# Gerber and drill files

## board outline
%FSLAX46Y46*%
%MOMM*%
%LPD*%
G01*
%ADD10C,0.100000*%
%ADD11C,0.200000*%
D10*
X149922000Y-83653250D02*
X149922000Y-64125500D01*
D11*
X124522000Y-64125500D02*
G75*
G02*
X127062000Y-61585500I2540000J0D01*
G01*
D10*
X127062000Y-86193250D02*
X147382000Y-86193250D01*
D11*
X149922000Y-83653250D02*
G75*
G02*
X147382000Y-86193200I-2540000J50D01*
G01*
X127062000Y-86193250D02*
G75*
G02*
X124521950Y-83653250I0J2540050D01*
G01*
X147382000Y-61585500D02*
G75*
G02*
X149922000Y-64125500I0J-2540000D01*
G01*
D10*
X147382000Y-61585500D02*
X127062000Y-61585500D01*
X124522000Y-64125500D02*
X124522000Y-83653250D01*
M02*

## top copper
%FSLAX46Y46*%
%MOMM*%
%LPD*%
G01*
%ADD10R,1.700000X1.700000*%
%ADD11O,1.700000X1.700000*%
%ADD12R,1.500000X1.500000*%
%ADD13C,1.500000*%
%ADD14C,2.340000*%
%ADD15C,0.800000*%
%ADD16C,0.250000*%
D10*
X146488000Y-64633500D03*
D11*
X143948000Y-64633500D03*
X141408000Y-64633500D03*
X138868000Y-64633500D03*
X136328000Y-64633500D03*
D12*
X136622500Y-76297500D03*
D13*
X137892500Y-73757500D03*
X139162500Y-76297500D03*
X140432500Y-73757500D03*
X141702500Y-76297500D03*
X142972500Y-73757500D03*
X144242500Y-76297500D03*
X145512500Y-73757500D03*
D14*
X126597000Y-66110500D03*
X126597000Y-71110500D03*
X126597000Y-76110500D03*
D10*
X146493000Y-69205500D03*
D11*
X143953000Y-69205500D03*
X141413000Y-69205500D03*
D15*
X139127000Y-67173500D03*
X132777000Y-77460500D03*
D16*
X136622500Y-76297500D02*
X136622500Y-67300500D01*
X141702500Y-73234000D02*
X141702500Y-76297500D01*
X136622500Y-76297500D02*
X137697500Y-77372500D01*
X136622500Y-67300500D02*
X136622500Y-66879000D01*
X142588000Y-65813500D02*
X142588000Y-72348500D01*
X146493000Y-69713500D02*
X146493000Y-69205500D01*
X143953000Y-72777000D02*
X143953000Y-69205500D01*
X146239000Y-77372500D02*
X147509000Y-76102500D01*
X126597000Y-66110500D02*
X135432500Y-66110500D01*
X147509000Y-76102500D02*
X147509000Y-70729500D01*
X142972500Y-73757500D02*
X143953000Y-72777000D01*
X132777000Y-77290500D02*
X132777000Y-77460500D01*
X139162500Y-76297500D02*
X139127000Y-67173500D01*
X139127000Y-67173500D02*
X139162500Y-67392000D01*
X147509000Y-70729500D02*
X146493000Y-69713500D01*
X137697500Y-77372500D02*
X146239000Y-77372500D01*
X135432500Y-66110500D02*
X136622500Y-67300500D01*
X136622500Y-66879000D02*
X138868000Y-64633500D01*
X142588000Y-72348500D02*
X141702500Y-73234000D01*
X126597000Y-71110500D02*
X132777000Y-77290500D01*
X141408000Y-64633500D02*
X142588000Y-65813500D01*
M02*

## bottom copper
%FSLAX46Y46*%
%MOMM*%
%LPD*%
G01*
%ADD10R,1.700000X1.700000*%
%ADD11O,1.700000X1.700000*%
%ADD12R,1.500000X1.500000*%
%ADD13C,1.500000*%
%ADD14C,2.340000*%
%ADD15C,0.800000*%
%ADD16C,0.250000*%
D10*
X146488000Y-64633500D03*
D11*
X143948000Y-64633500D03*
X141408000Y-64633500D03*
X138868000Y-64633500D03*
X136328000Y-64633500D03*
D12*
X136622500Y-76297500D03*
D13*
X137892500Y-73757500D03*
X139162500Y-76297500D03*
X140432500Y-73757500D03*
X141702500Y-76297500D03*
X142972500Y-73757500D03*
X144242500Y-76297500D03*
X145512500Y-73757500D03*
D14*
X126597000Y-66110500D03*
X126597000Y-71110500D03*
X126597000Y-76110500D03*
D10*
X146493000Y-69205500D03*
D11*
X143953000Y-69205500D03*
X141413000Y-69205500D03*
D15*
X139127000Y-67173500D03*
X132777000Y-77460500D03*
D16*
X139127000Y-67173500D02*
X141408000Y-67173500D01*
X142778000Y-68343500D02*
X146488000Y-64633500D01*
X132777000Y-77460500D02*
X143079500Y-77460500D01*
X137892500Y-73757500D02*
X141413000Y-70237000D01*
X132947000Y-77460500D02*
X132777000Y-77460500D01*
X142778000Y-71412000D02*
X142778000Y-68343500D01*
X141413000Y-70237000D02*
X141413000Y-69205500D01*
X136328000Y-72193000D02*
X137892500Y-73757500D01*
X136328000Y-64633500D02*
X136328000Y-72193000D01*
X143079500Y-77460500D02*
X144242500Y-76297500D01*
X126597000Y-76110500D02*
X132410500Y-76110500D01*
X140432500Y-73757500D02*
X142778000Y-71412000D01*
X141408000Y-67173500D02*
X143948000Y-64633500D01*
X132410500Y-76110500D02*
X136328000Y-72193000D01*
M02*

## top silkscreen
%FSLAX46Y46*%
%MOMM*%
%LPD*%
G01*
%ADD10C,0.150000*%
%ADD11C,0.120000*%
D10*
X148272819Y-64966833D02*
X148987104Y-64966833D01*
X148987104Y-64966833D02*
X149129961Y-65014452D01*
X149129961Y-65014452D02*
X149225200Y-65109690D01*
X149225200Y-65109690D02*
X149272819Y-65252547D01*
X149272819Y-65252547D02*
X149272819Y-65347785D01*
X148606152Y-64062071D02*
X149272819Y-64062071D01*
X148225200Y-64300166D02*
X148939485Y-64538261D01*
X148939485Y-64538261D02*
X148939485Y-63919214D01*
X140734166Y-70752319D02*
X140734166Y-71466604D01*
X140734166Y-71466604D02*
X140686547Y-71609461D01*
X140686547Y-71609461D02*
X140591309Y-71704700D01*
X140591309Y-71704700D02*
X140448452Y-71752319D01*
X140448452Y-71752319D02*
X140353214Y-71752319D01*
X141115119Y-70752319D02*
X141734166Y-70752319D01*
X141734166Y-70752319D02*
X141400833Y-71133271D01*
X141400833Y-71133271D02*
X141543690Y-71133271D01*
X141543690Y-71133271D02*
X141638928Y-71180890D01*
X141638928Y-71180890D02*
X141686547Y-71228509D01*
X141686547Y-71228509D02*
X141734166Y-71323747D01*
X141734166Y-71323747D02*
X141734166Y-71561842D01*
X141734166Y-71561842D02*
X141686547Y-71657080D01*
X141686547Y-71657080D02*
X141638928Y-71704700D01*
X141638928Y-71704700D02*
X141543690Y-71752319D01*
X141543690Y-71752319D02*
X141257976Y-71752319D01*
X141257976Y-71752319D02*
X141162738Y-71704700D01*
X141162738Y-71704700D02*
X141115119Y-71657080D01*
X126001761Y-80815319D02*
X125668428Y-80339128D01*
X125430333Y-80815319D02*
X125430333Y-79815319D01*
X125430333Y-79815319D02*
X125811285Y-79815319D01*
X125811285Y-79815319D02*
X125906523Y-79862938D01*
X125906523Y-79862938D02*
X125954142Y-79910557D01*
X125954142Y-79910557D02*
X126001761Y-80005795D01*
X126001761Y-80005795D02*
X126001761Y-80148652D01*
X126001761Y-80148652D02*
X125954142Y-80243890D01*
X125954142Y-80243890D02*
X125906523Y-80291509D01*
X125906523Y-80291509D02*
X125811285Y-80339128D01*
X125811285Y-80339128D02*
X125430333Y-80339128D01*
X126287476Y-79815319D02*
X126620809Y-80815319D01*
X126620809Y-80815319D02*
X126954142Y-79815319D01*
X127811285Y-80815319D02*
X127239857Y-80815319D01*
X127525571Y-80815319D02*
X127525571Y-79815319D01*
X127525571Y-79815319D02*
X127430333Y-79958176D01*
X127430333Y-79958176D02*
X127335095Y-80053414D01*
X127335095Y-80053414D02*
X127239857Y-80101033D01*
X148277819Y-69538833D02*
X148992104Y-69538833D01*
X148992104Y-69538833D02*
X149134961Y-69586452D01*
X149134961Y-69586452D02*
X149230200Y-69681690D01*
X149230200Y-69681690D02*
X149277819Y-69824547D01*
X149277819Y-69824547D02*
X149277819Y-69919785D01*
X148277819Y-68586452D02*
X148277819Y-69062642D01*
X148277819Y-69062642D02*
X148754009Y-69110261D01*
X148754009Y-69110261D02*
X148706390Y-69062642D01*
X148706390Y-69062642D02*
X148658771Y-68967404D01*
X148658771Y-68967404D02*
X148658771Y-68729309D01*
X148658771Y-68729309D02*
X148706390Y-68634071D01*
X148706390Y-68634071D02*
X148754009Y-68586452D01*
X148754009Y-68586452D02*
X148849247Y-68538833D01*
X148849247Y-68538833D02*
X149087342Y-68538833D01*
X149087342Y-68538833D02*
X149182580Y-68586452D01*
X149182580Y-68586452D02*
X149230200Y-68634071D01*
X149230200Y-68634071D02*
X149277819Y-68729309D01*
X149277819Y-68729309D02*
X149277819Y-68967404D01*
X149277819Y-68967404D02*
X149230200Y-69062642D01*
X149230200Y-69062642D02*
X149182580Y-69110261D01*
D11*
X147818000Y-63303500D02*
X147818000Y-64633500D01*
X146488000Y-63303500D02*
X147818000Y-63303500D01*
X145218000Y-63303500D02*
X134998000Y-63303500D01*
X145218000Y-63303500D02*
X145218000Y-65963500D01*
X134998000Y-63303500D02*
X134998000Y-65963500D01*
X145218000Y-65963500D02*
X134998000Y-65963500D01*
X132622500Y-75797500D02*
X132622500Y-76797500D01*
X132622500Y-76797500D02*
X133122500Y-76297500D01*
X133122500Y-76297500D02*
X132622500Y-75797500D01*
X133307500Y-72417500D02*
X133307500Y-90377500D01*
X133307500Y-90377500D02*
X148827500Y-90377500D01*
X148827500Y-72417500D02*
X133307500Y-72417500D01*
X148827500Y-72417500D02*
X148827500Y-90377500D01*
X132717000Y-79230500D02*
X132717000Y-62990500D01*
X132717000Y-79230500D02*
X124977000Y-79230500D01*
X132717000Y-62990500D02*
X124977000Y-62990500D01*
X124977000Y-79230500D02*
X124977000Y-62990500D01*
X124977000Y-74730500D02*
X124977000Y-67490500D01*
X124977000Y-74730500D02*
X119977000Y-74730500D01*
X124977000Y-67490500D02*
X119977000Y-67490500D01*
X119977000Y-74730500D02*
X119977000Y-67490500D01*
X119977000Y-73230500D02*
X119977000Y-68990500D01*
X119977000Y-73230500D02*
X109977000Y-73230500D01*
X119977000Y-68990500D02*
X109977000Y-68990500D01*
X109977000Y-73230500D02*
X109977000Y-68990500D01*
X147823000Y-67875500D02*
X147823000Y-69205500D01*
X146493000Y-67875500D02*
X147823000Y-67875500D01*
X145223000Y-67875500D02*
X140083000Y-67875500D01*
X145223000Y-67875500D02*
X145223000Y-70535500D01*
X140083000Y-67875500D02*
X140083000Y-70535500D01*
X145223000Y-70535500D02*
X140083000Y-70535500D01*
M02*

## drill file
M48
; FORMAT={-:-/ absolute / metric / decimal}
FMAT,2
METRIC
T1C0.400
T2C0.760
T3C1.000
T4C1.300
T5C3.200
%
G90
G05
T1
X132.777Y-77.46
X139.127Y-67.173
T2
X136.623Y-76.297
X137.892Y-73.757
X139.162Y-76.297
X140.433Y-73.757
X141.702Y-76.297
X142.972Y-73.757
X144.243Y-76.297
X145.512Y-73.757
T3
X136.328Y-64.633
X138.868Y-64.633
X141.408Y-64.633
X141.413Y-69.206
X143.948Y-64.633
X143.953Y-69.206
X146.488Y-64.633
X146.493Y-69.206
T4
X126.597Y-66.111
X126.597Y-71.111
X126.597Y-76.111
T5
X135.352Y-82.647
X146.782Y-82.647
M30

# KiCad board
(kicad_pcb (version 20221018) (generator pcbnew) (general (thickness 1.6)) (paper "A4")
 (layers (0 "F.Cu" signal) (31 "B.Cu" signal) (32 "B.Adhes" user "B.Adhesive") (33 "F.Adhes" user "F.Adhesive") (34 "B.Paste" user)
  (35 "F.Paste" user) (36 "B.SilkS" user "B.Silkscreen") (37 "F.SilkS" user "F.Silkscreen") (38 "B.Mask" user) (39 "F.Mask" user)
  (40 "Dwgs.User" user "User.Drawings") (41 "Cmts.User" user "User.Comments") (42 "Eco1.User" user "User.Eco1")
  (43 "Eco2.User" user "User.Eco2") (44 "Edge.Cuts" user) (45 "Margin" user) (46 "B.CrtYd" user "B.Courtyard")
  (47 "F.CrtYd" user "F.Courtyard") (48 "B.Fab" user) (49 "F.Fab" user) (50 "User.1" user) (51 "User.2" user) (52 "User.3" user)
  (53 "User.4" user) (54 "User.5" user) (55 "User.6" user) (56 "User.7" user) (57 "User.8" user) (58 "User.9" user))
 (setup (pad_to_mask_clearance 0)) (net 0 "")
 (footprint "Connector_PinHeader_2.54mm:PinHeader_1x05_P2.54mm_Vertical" (layer "F.Cu") (at 146.488 64.6335 -90)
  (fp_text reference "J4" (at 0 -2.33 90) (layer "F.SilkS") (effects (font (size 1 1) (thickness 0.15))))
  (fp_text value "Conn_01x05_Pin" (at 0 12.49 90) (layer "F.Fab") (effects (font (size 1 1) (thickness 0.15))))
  (fp_line (start -1.33 -1.33) (end 0 -1.33) (stroke (width 0.12) (type solid)) (layer "F.SilkS"))
  (fp_line (start -1.33 0) (end -1.33 -1.33) (stroke (width 0.12) (type solid)) (layer "F.SilkS"))
  (fp_line (start -1.33 1.27) (end -1.33 11.49) (stroke (width 0.12) (type solid)) (layer "F.SilkS"))
  (fp_line (start -1.33 1.27) (end 1.33 1.27) (stroke (width 0.12) (type solid)) (layer "F.SilkS"))
  (fp_line (start -1.33 11.49) (end 1.33 11.49) (stroke (width 0.12) (type solid)) (layer "F.SilkS"))
  (fp_line (start 1.33 1.27) (end 1.33 11.49) (stroke (width 0.12) (type solid)) (layer "F.SilkS"))
  (pad "1" thru_hole rect (at 0 0 270) (size 1.7 1.7) (drill 1) (layers "*.Cu" "*.Mask"))
  (pad "2" thru_hole oval (at 0 2.54 270) (size 1.7 1.7) (drill 1) (layers "*.Cu" "*.Mask"))
  (pad "3" thru_hole oval (at 0 5.08 270) (size 1.7 1.7) (drill 1) (layers "*.Cu" "*.Mask"))
  (pad "4" thru_hole oval (at 0 7.62 270) (size 1.7 1.7) (drill 1) (layers "*.Cu" "*.Mask"))
  (pad "5" thru_hole oval (at 0 10.16 270) (size 1.7 1.7) (drill 1) (layers "*.Cu" "*.Mask")))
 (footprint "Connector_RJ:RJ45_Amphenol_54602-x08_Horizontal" (layer "F.Cu") (at 136.6225 76.2975)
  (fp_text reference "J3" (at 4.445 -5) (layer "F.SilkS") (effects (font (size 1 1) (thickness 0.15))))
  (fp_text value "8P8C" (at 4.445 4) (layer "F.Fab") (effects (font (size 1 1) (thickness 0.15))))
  (fp_line (start -4 -0.5) (end -4 0.5) (stroke (width 0.12) (type solid)) (layer "F.SilkS"))
  (fp_line (start -4 0.5) (end -3.5 0) (stroke (width 0.12) (type solid)) (layer "F.SilkS"))
  (fp_line (start -3.5 0) (end -4 -0.5) (stroke (width 0.12) (type solid)) (layer "F.SilkS"))
  (fp_line (start -3.315 -3.88) (end -3.315 14.08) (stroke (width 0.12) (type solid)) (layer "F.SilkS"))
  (fp_line (start -3.315 14.08) (end 12.205 14.08) (stroke (width 0.12) (type solid)) (layer "F.SilkS"))
  (fp_line (start 12.205 -3.88) (end -3.315 -3.88) (stroke (width 0.12) (type solid)) (layer "F.SilkS"))
  (fp_line (start 12.205 -3.88) (end 12.205 14.08) (stroke (width 0.12) (type solid)) (layer "F.SilkS"))
  (pad "" np_thru_hole circle (at -1.27 6.35) (size 3.2 3.2) (drill 3.2) (layers "F&B.Cu" "*.Mask"))
  (pad "" np_thru_hole circle (at 10.16 6.35) (size 3.2 3.2) (drill 3.2) (layers "F&B.Cu" "*.Mask"))
  (pad "1" thru_hole rect (at 0 0) (size 1.5 1.5) (drill 0.76) (layers "*.Cu" "*.Mask"))
  (pad "2" thru_hole circle (at 1.27 -2.54) (size 1.5 1.5) (drill 0.76) (layers "*.Cu" "*.Mask"))
  (pad "3" thru_hole circle (at 2.54 0) (size 1.5 1.5) (drill 0.76) (layers "*.Cu" "*.Mask"))
  (pad "4" thru_hole circle (at 3.81 -2.54) (size 1.5 1.5) (drill 0.76) (layers "*.Cu" "*.Mask"))
  (pad "5" thru_hole circle (at 5.08 0) (size 1.5 1.5) (drill 0.76) (layers "*.Cu" "*.Mask"))
  (pad "6" thru_hole circle (at 6.35 -2.54) (size 1.5 1.5) (drill 0.76) (layers "*.Cu" "*.Mask"))
  (pad "7" thru_hole circle (at 7.62 0) (size 1.5 1.5) (drill 0.76) (layers "*.Cu" "*.Mask"))
  (pad "8" thru_hole circle (at 8.89 -2.54) (size 1.5 1.5) (drill 0.76) (layers "*.Cu" "*.Mask")))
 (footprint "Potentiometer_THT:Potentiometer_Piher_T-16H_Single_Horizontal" (layer "F.Cu") (at 126.597 66.1105 180)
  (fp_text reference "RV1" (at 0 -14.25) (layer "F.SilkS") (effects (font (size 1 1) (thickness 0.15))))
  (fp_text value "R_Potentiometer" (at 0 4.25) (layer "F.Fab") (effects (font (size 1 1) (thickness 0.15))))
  (fp_line (start -6.12 -13.12) (end -6.12 3.12) (stroke (width 0.12) (type solid)) (layer "F.SilkS"))
  (fp_line (start -6.12 -13.12) (end 1.62 -13.12) (stroke (width 0.12) (type solid)) (layer "F.SilkS"))
  (fp_line (start -6.12 3.12) (end 1.62 3.12) (stroke (width 0.12) (type solid)) (layer "F.SilkS"))
  (fp_line (start 1.62 -13.12) (end 1.62 3.12) (stroke (width 0.12) (type solid)) (layer "F.SilkS"))
  (fp_line (start 1.62 -8.62) (end 1.62 -1.38) (stroke (width 0.12) (type solid)) (layer "F.SilkS"))
  (fp_line (start 1.62 -8.62) (end 6.62 -8.62) (stroke (width 0.12) (type solid)) (layer "F.SilkS"))
  (fp_line (start 1.62 -1.38) (end 6.62 -1.38) (stroke (width 0.12) (type solid)) (layer "F.SilkS"))
  (fp_line (start 6.62 -8.62) (end 6.62 -1.38) (stroke (width 0.12) (type solid)) (layer "F.SilkS"))
  (fp_line (start 6.62 -7.12) (end 6.62 -2.88) (stroke (width 0.12) (type solid)) (layer "F.SilkS"))
  (fp_line (start 6.62 -7.12) (end 16.62 -7.12) (stroke (width 0.12) (type solid)) (layer "F.SilkS"))
  (fp_line (start 6.62 -2.88) (end 16.62 -2.88) (stroke (width 0.12) (type solid)) (layer "F.SilkS"))
  (fp_line (start 16.62 -7.12) (end 16.62 -2.88) (stroke (width 0.12) (type solid)) (layer "F.SilkS"))
  (pad "1" thru_hole circle (at 0 0 180) (size 2.34 2.34) (drill 1.3) (layers "*.Cu" "*.Mask"))
  (pad "2" thru_hole circle (at 0 -5 180) (size 2.34 2.34) (drill 1.3) (layers "*.Cu" "*.Mask"))
  (pad "3" thru_hole circle (at 0 -10 180) (size 2.34 2.34) (drill 1.3) (layers "*.Cu" "*.Mask")))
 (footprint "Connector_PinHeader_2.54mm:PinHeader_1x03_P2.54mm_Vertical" (layer "F.Cu") (at 146.493 69.2055 -90)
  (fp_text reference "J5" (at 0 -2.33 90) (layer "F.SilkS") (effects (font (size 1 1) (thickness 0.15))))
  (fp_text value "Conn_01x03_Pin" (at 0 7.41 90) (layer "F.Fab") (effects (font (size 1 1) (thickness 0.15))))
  (fp_line (start -1.33 -1.33) (end 0 -1.33) (stroke (width 0.12) (type solid)) (layer "F.SilkS"))
  (fp_line (start -1.33 0) (end -1.33 -1.33) (stroke (width 0.12) (type solid)) (layer "F.SilkS"))
  (fp_line (start -1.33 1.27) (end -1.33 6.41) (stroke (width 0.12) (type solid)) (layer "F.SilkS"))
  (fp_line (start -1.33 1.27) (end 1.33 1.27) (stroke (width 0.12) (type solid)) (layer "F.SilkS"))
  (fp_line (start -1.33 6.41) (end 1.33 6.41) (stroke (width 0.12) (type solid)) (layer "F.SilkS"))
  (fp_line (start 1.33 1.27) (end 1.33 6.41) (stroke (width 0.12) (type solid)) (layer "F.SilkS"))
  (pad "1" thru_hole rect (at 0 0 270) (size 1.7 1.7) (drill 1) (layers "*.Cu" "*.Mask"))
  (pad "2" thru_hole oval (at 0 2.54 270) (size 1.7 1.7) (drill 1) (layers "*.Cu" "*.Mask"))
  (pad "3" thru_hole oval (at 0 5.08 270) (size 1.7 1.7) (drill 1) (layers "*.Cu" "*.Mask")))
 (gr_line (start 149.922 83.65325) (end 149.922 64.1255) (stroke (width 0.1) (type default)) (layer "Edge.Cuts"))
 (gr_arc (start 124.522 64.1255) (mid 125.265949 62.329449) (end 127.062 61.5855) (stroke (width 0.2) (type default)) (layer "Edge.Cuts"))
 (gr_line (start 127.062 86.19325) (end 147.382 86.19325) (stroke (width 0.1) (type default)) (layer "Edge.Cuts"))
 (gr_arc (start 149.922 83.65325) (mid 149.178051 85.449301) (end 147.382 86.19325) (stroke (width 0.2) (type default)) (layer "Edge.Cuts"))
 (gr_arc (start 127.062 86.19325) (mid 125.265949 85.449301) (end 124.522 83.65325) (stroke (width 0.2) (type default)) (layer "Edge.Cuts"))
 (gr_arc (start 147.382 61.5855) (mid 149.178063 62.329437) (end 149.922 64.1255) (stroke (width 0.2) (type default)) (layer "Edge.Cuts"))
 (gr_line (start 147.382 61.5855) (end 127.062 61.5855) (stroke (width 0.1) (type default)) (layer "Edge.Cuts"))
 (gr_line (start 124.522 64.1255) (end 124.522 83.65325) (stroke (width 0.1) (type default)) (layer "Edge.Cuts"))
 (segment (start 136.6225 76.2975) (end 136.6225 67.3005) (width 0.25) (layer "F.Cu") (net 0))
 (segment (start 141.7025 73.234) (end 141.7025 76.2975) (width 0.25) (layer "F.Cu") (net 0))
 (segment (start 136.6225 76.2975) (end 137.6975 77.3725) (width 0.25) (layer "F.Cu") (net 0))
 (segment (start 136.6225 67.3005) (end 136.6225 66.879) (width 0.25) (layer "F.Cu") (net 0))
 (segment (start 142.588 65.8135) (end 142.588 72.3485) (width 0.25) (layer "F.Cu") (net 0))
 (segment (start 146.493 69.7135) (end 146.493 69.2055) (width 0.25) (layer "F.Cu") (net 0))
 (segment (start 143.953 72.777) (end 143.953 69.2055) (width 0.25) (layer "F.Cu") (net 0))
 (segment (start 146.239 77.3725) (end 147.509 76.1025) (width 0.25) (layer "F.Cu") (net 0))
 (segment (start 126.597 66.1105) (end 135.4325 66.1105) (width 0.25) (layer "F.Cu") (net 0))
 (segment (start 147.509 76.1025) (end 147.509 70.7295) (width 0.25) (layer "F.Cu") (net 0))
 (segment (start 142.9725 73.7575) (end 143.953 72.777) (width 0.25) (layer "F.Cu") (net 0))
 (segment (start 132.777 77.2905) (end 132.777 77.4605) (width 0.25) (layer "F.Cu") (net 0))
 (segment (start 139.1625 76.2975) (end 139.127 67.1735) (width 0.25) (layer "F.Cu") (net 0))
 (segment (start 139.127 67.1735) (end 139.1625 67.392) (width 0.25) (layer "F.Cu") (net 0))
 (segment (start 147.509 70.7295) (end 146.493 69.7135) (width 0.25) (layer "F.Cu") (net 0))
 (segment (start 137.6975 77.3725) (end 146.239 77.3725) (width 0.25) (layer "F.Cu") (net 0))
 (segment (start 135.4325 66.1105) (end 136.6225 67.3005) (width 0.25) (layer "F.Cu") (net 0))
 (segment (start 136.6225 66.879) (end 138.868 64.6335) (width 0.25) (layer "F.Cu") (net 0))
 (segment (start 142.588 72.3485) (end 141.7025 73.234) (width 0.25) (layer "F.Cu") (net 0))
 (segment (start 126.597 71.1105) (end 132.777 77.2905) (width 0.25) (layer "F.Cu") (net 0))
 (segment (start 141.408 64.6335) (end 142.588 65.8135) (width 0.25) (layer "F.Cu") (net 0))
 (via (at 139.127 67.1735) (size 0.8) (drill 0.4) (layers "F.Cu" "B.Cu") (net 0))
 (via (at 132.777 77.4605) (size 0.8) (drill 0.4) (layers "F.Cu" "B.Cu") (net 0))
 (segment (start 139.127 67.1735) (end 141.408 67.1735) (width 0.25) (layer "B.Cu") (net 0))
 (segment (start 142.778 68.3435) (end 146.488 64.6335) (width 0.25) (layer "B.Cu") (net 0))
 (segment (start 132.777 77.4605) (end 143.0795 77.4605) (width 0.25) (layer "B.Cu") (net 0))
 (segment (start 137.8925 73.7575) (end 141.413 70.237) (width 0.25) (layer "B.Cu") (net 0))
 (segment (start 132.947 77.4605) (end 132.777 77.4605) (width 0.25) (layer "B.Cu") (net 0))
 (segment (start 142.778 71.412) (end 142.778 68.3435) (width 0.25) (layer "B.Cu") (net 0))
 (segment (start 141.413 70.237) (end 141.413 69.2055) (width 0.25) (layer "B.Cu") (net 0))
 (segment (start 136.328 72.193) (end 137.8925 73.7575) (width 0.25) (layer "B.Cu") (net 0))
 (segment (start 136.328 64.6335) (end 136.328 72.193) (width 0.25) (layer "B.Cu") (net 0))
 (segment (start 143.0795 77.4605) (end 144.2425 76.2975) (width 0.25) (layer "B.Cu") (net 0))
 (segment (start 126.597 76.1105) (end 132.4105 76.1105) (width 0.25) (layer "B.Cu") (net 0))
 (segment (start 140.4325 73.7575) (end 142.778 71.412) (width 0.25) (layer "B.Cu") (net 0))
 (segment (start 141.408 67.1735) (end 143.948 64.6335) (width 0.25) (layer "B.Cu") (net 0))
 (segment (start 132.4105 76.1105) (end 136.328 72.193) (width 0.25) (layer "B.Cu") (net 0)))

